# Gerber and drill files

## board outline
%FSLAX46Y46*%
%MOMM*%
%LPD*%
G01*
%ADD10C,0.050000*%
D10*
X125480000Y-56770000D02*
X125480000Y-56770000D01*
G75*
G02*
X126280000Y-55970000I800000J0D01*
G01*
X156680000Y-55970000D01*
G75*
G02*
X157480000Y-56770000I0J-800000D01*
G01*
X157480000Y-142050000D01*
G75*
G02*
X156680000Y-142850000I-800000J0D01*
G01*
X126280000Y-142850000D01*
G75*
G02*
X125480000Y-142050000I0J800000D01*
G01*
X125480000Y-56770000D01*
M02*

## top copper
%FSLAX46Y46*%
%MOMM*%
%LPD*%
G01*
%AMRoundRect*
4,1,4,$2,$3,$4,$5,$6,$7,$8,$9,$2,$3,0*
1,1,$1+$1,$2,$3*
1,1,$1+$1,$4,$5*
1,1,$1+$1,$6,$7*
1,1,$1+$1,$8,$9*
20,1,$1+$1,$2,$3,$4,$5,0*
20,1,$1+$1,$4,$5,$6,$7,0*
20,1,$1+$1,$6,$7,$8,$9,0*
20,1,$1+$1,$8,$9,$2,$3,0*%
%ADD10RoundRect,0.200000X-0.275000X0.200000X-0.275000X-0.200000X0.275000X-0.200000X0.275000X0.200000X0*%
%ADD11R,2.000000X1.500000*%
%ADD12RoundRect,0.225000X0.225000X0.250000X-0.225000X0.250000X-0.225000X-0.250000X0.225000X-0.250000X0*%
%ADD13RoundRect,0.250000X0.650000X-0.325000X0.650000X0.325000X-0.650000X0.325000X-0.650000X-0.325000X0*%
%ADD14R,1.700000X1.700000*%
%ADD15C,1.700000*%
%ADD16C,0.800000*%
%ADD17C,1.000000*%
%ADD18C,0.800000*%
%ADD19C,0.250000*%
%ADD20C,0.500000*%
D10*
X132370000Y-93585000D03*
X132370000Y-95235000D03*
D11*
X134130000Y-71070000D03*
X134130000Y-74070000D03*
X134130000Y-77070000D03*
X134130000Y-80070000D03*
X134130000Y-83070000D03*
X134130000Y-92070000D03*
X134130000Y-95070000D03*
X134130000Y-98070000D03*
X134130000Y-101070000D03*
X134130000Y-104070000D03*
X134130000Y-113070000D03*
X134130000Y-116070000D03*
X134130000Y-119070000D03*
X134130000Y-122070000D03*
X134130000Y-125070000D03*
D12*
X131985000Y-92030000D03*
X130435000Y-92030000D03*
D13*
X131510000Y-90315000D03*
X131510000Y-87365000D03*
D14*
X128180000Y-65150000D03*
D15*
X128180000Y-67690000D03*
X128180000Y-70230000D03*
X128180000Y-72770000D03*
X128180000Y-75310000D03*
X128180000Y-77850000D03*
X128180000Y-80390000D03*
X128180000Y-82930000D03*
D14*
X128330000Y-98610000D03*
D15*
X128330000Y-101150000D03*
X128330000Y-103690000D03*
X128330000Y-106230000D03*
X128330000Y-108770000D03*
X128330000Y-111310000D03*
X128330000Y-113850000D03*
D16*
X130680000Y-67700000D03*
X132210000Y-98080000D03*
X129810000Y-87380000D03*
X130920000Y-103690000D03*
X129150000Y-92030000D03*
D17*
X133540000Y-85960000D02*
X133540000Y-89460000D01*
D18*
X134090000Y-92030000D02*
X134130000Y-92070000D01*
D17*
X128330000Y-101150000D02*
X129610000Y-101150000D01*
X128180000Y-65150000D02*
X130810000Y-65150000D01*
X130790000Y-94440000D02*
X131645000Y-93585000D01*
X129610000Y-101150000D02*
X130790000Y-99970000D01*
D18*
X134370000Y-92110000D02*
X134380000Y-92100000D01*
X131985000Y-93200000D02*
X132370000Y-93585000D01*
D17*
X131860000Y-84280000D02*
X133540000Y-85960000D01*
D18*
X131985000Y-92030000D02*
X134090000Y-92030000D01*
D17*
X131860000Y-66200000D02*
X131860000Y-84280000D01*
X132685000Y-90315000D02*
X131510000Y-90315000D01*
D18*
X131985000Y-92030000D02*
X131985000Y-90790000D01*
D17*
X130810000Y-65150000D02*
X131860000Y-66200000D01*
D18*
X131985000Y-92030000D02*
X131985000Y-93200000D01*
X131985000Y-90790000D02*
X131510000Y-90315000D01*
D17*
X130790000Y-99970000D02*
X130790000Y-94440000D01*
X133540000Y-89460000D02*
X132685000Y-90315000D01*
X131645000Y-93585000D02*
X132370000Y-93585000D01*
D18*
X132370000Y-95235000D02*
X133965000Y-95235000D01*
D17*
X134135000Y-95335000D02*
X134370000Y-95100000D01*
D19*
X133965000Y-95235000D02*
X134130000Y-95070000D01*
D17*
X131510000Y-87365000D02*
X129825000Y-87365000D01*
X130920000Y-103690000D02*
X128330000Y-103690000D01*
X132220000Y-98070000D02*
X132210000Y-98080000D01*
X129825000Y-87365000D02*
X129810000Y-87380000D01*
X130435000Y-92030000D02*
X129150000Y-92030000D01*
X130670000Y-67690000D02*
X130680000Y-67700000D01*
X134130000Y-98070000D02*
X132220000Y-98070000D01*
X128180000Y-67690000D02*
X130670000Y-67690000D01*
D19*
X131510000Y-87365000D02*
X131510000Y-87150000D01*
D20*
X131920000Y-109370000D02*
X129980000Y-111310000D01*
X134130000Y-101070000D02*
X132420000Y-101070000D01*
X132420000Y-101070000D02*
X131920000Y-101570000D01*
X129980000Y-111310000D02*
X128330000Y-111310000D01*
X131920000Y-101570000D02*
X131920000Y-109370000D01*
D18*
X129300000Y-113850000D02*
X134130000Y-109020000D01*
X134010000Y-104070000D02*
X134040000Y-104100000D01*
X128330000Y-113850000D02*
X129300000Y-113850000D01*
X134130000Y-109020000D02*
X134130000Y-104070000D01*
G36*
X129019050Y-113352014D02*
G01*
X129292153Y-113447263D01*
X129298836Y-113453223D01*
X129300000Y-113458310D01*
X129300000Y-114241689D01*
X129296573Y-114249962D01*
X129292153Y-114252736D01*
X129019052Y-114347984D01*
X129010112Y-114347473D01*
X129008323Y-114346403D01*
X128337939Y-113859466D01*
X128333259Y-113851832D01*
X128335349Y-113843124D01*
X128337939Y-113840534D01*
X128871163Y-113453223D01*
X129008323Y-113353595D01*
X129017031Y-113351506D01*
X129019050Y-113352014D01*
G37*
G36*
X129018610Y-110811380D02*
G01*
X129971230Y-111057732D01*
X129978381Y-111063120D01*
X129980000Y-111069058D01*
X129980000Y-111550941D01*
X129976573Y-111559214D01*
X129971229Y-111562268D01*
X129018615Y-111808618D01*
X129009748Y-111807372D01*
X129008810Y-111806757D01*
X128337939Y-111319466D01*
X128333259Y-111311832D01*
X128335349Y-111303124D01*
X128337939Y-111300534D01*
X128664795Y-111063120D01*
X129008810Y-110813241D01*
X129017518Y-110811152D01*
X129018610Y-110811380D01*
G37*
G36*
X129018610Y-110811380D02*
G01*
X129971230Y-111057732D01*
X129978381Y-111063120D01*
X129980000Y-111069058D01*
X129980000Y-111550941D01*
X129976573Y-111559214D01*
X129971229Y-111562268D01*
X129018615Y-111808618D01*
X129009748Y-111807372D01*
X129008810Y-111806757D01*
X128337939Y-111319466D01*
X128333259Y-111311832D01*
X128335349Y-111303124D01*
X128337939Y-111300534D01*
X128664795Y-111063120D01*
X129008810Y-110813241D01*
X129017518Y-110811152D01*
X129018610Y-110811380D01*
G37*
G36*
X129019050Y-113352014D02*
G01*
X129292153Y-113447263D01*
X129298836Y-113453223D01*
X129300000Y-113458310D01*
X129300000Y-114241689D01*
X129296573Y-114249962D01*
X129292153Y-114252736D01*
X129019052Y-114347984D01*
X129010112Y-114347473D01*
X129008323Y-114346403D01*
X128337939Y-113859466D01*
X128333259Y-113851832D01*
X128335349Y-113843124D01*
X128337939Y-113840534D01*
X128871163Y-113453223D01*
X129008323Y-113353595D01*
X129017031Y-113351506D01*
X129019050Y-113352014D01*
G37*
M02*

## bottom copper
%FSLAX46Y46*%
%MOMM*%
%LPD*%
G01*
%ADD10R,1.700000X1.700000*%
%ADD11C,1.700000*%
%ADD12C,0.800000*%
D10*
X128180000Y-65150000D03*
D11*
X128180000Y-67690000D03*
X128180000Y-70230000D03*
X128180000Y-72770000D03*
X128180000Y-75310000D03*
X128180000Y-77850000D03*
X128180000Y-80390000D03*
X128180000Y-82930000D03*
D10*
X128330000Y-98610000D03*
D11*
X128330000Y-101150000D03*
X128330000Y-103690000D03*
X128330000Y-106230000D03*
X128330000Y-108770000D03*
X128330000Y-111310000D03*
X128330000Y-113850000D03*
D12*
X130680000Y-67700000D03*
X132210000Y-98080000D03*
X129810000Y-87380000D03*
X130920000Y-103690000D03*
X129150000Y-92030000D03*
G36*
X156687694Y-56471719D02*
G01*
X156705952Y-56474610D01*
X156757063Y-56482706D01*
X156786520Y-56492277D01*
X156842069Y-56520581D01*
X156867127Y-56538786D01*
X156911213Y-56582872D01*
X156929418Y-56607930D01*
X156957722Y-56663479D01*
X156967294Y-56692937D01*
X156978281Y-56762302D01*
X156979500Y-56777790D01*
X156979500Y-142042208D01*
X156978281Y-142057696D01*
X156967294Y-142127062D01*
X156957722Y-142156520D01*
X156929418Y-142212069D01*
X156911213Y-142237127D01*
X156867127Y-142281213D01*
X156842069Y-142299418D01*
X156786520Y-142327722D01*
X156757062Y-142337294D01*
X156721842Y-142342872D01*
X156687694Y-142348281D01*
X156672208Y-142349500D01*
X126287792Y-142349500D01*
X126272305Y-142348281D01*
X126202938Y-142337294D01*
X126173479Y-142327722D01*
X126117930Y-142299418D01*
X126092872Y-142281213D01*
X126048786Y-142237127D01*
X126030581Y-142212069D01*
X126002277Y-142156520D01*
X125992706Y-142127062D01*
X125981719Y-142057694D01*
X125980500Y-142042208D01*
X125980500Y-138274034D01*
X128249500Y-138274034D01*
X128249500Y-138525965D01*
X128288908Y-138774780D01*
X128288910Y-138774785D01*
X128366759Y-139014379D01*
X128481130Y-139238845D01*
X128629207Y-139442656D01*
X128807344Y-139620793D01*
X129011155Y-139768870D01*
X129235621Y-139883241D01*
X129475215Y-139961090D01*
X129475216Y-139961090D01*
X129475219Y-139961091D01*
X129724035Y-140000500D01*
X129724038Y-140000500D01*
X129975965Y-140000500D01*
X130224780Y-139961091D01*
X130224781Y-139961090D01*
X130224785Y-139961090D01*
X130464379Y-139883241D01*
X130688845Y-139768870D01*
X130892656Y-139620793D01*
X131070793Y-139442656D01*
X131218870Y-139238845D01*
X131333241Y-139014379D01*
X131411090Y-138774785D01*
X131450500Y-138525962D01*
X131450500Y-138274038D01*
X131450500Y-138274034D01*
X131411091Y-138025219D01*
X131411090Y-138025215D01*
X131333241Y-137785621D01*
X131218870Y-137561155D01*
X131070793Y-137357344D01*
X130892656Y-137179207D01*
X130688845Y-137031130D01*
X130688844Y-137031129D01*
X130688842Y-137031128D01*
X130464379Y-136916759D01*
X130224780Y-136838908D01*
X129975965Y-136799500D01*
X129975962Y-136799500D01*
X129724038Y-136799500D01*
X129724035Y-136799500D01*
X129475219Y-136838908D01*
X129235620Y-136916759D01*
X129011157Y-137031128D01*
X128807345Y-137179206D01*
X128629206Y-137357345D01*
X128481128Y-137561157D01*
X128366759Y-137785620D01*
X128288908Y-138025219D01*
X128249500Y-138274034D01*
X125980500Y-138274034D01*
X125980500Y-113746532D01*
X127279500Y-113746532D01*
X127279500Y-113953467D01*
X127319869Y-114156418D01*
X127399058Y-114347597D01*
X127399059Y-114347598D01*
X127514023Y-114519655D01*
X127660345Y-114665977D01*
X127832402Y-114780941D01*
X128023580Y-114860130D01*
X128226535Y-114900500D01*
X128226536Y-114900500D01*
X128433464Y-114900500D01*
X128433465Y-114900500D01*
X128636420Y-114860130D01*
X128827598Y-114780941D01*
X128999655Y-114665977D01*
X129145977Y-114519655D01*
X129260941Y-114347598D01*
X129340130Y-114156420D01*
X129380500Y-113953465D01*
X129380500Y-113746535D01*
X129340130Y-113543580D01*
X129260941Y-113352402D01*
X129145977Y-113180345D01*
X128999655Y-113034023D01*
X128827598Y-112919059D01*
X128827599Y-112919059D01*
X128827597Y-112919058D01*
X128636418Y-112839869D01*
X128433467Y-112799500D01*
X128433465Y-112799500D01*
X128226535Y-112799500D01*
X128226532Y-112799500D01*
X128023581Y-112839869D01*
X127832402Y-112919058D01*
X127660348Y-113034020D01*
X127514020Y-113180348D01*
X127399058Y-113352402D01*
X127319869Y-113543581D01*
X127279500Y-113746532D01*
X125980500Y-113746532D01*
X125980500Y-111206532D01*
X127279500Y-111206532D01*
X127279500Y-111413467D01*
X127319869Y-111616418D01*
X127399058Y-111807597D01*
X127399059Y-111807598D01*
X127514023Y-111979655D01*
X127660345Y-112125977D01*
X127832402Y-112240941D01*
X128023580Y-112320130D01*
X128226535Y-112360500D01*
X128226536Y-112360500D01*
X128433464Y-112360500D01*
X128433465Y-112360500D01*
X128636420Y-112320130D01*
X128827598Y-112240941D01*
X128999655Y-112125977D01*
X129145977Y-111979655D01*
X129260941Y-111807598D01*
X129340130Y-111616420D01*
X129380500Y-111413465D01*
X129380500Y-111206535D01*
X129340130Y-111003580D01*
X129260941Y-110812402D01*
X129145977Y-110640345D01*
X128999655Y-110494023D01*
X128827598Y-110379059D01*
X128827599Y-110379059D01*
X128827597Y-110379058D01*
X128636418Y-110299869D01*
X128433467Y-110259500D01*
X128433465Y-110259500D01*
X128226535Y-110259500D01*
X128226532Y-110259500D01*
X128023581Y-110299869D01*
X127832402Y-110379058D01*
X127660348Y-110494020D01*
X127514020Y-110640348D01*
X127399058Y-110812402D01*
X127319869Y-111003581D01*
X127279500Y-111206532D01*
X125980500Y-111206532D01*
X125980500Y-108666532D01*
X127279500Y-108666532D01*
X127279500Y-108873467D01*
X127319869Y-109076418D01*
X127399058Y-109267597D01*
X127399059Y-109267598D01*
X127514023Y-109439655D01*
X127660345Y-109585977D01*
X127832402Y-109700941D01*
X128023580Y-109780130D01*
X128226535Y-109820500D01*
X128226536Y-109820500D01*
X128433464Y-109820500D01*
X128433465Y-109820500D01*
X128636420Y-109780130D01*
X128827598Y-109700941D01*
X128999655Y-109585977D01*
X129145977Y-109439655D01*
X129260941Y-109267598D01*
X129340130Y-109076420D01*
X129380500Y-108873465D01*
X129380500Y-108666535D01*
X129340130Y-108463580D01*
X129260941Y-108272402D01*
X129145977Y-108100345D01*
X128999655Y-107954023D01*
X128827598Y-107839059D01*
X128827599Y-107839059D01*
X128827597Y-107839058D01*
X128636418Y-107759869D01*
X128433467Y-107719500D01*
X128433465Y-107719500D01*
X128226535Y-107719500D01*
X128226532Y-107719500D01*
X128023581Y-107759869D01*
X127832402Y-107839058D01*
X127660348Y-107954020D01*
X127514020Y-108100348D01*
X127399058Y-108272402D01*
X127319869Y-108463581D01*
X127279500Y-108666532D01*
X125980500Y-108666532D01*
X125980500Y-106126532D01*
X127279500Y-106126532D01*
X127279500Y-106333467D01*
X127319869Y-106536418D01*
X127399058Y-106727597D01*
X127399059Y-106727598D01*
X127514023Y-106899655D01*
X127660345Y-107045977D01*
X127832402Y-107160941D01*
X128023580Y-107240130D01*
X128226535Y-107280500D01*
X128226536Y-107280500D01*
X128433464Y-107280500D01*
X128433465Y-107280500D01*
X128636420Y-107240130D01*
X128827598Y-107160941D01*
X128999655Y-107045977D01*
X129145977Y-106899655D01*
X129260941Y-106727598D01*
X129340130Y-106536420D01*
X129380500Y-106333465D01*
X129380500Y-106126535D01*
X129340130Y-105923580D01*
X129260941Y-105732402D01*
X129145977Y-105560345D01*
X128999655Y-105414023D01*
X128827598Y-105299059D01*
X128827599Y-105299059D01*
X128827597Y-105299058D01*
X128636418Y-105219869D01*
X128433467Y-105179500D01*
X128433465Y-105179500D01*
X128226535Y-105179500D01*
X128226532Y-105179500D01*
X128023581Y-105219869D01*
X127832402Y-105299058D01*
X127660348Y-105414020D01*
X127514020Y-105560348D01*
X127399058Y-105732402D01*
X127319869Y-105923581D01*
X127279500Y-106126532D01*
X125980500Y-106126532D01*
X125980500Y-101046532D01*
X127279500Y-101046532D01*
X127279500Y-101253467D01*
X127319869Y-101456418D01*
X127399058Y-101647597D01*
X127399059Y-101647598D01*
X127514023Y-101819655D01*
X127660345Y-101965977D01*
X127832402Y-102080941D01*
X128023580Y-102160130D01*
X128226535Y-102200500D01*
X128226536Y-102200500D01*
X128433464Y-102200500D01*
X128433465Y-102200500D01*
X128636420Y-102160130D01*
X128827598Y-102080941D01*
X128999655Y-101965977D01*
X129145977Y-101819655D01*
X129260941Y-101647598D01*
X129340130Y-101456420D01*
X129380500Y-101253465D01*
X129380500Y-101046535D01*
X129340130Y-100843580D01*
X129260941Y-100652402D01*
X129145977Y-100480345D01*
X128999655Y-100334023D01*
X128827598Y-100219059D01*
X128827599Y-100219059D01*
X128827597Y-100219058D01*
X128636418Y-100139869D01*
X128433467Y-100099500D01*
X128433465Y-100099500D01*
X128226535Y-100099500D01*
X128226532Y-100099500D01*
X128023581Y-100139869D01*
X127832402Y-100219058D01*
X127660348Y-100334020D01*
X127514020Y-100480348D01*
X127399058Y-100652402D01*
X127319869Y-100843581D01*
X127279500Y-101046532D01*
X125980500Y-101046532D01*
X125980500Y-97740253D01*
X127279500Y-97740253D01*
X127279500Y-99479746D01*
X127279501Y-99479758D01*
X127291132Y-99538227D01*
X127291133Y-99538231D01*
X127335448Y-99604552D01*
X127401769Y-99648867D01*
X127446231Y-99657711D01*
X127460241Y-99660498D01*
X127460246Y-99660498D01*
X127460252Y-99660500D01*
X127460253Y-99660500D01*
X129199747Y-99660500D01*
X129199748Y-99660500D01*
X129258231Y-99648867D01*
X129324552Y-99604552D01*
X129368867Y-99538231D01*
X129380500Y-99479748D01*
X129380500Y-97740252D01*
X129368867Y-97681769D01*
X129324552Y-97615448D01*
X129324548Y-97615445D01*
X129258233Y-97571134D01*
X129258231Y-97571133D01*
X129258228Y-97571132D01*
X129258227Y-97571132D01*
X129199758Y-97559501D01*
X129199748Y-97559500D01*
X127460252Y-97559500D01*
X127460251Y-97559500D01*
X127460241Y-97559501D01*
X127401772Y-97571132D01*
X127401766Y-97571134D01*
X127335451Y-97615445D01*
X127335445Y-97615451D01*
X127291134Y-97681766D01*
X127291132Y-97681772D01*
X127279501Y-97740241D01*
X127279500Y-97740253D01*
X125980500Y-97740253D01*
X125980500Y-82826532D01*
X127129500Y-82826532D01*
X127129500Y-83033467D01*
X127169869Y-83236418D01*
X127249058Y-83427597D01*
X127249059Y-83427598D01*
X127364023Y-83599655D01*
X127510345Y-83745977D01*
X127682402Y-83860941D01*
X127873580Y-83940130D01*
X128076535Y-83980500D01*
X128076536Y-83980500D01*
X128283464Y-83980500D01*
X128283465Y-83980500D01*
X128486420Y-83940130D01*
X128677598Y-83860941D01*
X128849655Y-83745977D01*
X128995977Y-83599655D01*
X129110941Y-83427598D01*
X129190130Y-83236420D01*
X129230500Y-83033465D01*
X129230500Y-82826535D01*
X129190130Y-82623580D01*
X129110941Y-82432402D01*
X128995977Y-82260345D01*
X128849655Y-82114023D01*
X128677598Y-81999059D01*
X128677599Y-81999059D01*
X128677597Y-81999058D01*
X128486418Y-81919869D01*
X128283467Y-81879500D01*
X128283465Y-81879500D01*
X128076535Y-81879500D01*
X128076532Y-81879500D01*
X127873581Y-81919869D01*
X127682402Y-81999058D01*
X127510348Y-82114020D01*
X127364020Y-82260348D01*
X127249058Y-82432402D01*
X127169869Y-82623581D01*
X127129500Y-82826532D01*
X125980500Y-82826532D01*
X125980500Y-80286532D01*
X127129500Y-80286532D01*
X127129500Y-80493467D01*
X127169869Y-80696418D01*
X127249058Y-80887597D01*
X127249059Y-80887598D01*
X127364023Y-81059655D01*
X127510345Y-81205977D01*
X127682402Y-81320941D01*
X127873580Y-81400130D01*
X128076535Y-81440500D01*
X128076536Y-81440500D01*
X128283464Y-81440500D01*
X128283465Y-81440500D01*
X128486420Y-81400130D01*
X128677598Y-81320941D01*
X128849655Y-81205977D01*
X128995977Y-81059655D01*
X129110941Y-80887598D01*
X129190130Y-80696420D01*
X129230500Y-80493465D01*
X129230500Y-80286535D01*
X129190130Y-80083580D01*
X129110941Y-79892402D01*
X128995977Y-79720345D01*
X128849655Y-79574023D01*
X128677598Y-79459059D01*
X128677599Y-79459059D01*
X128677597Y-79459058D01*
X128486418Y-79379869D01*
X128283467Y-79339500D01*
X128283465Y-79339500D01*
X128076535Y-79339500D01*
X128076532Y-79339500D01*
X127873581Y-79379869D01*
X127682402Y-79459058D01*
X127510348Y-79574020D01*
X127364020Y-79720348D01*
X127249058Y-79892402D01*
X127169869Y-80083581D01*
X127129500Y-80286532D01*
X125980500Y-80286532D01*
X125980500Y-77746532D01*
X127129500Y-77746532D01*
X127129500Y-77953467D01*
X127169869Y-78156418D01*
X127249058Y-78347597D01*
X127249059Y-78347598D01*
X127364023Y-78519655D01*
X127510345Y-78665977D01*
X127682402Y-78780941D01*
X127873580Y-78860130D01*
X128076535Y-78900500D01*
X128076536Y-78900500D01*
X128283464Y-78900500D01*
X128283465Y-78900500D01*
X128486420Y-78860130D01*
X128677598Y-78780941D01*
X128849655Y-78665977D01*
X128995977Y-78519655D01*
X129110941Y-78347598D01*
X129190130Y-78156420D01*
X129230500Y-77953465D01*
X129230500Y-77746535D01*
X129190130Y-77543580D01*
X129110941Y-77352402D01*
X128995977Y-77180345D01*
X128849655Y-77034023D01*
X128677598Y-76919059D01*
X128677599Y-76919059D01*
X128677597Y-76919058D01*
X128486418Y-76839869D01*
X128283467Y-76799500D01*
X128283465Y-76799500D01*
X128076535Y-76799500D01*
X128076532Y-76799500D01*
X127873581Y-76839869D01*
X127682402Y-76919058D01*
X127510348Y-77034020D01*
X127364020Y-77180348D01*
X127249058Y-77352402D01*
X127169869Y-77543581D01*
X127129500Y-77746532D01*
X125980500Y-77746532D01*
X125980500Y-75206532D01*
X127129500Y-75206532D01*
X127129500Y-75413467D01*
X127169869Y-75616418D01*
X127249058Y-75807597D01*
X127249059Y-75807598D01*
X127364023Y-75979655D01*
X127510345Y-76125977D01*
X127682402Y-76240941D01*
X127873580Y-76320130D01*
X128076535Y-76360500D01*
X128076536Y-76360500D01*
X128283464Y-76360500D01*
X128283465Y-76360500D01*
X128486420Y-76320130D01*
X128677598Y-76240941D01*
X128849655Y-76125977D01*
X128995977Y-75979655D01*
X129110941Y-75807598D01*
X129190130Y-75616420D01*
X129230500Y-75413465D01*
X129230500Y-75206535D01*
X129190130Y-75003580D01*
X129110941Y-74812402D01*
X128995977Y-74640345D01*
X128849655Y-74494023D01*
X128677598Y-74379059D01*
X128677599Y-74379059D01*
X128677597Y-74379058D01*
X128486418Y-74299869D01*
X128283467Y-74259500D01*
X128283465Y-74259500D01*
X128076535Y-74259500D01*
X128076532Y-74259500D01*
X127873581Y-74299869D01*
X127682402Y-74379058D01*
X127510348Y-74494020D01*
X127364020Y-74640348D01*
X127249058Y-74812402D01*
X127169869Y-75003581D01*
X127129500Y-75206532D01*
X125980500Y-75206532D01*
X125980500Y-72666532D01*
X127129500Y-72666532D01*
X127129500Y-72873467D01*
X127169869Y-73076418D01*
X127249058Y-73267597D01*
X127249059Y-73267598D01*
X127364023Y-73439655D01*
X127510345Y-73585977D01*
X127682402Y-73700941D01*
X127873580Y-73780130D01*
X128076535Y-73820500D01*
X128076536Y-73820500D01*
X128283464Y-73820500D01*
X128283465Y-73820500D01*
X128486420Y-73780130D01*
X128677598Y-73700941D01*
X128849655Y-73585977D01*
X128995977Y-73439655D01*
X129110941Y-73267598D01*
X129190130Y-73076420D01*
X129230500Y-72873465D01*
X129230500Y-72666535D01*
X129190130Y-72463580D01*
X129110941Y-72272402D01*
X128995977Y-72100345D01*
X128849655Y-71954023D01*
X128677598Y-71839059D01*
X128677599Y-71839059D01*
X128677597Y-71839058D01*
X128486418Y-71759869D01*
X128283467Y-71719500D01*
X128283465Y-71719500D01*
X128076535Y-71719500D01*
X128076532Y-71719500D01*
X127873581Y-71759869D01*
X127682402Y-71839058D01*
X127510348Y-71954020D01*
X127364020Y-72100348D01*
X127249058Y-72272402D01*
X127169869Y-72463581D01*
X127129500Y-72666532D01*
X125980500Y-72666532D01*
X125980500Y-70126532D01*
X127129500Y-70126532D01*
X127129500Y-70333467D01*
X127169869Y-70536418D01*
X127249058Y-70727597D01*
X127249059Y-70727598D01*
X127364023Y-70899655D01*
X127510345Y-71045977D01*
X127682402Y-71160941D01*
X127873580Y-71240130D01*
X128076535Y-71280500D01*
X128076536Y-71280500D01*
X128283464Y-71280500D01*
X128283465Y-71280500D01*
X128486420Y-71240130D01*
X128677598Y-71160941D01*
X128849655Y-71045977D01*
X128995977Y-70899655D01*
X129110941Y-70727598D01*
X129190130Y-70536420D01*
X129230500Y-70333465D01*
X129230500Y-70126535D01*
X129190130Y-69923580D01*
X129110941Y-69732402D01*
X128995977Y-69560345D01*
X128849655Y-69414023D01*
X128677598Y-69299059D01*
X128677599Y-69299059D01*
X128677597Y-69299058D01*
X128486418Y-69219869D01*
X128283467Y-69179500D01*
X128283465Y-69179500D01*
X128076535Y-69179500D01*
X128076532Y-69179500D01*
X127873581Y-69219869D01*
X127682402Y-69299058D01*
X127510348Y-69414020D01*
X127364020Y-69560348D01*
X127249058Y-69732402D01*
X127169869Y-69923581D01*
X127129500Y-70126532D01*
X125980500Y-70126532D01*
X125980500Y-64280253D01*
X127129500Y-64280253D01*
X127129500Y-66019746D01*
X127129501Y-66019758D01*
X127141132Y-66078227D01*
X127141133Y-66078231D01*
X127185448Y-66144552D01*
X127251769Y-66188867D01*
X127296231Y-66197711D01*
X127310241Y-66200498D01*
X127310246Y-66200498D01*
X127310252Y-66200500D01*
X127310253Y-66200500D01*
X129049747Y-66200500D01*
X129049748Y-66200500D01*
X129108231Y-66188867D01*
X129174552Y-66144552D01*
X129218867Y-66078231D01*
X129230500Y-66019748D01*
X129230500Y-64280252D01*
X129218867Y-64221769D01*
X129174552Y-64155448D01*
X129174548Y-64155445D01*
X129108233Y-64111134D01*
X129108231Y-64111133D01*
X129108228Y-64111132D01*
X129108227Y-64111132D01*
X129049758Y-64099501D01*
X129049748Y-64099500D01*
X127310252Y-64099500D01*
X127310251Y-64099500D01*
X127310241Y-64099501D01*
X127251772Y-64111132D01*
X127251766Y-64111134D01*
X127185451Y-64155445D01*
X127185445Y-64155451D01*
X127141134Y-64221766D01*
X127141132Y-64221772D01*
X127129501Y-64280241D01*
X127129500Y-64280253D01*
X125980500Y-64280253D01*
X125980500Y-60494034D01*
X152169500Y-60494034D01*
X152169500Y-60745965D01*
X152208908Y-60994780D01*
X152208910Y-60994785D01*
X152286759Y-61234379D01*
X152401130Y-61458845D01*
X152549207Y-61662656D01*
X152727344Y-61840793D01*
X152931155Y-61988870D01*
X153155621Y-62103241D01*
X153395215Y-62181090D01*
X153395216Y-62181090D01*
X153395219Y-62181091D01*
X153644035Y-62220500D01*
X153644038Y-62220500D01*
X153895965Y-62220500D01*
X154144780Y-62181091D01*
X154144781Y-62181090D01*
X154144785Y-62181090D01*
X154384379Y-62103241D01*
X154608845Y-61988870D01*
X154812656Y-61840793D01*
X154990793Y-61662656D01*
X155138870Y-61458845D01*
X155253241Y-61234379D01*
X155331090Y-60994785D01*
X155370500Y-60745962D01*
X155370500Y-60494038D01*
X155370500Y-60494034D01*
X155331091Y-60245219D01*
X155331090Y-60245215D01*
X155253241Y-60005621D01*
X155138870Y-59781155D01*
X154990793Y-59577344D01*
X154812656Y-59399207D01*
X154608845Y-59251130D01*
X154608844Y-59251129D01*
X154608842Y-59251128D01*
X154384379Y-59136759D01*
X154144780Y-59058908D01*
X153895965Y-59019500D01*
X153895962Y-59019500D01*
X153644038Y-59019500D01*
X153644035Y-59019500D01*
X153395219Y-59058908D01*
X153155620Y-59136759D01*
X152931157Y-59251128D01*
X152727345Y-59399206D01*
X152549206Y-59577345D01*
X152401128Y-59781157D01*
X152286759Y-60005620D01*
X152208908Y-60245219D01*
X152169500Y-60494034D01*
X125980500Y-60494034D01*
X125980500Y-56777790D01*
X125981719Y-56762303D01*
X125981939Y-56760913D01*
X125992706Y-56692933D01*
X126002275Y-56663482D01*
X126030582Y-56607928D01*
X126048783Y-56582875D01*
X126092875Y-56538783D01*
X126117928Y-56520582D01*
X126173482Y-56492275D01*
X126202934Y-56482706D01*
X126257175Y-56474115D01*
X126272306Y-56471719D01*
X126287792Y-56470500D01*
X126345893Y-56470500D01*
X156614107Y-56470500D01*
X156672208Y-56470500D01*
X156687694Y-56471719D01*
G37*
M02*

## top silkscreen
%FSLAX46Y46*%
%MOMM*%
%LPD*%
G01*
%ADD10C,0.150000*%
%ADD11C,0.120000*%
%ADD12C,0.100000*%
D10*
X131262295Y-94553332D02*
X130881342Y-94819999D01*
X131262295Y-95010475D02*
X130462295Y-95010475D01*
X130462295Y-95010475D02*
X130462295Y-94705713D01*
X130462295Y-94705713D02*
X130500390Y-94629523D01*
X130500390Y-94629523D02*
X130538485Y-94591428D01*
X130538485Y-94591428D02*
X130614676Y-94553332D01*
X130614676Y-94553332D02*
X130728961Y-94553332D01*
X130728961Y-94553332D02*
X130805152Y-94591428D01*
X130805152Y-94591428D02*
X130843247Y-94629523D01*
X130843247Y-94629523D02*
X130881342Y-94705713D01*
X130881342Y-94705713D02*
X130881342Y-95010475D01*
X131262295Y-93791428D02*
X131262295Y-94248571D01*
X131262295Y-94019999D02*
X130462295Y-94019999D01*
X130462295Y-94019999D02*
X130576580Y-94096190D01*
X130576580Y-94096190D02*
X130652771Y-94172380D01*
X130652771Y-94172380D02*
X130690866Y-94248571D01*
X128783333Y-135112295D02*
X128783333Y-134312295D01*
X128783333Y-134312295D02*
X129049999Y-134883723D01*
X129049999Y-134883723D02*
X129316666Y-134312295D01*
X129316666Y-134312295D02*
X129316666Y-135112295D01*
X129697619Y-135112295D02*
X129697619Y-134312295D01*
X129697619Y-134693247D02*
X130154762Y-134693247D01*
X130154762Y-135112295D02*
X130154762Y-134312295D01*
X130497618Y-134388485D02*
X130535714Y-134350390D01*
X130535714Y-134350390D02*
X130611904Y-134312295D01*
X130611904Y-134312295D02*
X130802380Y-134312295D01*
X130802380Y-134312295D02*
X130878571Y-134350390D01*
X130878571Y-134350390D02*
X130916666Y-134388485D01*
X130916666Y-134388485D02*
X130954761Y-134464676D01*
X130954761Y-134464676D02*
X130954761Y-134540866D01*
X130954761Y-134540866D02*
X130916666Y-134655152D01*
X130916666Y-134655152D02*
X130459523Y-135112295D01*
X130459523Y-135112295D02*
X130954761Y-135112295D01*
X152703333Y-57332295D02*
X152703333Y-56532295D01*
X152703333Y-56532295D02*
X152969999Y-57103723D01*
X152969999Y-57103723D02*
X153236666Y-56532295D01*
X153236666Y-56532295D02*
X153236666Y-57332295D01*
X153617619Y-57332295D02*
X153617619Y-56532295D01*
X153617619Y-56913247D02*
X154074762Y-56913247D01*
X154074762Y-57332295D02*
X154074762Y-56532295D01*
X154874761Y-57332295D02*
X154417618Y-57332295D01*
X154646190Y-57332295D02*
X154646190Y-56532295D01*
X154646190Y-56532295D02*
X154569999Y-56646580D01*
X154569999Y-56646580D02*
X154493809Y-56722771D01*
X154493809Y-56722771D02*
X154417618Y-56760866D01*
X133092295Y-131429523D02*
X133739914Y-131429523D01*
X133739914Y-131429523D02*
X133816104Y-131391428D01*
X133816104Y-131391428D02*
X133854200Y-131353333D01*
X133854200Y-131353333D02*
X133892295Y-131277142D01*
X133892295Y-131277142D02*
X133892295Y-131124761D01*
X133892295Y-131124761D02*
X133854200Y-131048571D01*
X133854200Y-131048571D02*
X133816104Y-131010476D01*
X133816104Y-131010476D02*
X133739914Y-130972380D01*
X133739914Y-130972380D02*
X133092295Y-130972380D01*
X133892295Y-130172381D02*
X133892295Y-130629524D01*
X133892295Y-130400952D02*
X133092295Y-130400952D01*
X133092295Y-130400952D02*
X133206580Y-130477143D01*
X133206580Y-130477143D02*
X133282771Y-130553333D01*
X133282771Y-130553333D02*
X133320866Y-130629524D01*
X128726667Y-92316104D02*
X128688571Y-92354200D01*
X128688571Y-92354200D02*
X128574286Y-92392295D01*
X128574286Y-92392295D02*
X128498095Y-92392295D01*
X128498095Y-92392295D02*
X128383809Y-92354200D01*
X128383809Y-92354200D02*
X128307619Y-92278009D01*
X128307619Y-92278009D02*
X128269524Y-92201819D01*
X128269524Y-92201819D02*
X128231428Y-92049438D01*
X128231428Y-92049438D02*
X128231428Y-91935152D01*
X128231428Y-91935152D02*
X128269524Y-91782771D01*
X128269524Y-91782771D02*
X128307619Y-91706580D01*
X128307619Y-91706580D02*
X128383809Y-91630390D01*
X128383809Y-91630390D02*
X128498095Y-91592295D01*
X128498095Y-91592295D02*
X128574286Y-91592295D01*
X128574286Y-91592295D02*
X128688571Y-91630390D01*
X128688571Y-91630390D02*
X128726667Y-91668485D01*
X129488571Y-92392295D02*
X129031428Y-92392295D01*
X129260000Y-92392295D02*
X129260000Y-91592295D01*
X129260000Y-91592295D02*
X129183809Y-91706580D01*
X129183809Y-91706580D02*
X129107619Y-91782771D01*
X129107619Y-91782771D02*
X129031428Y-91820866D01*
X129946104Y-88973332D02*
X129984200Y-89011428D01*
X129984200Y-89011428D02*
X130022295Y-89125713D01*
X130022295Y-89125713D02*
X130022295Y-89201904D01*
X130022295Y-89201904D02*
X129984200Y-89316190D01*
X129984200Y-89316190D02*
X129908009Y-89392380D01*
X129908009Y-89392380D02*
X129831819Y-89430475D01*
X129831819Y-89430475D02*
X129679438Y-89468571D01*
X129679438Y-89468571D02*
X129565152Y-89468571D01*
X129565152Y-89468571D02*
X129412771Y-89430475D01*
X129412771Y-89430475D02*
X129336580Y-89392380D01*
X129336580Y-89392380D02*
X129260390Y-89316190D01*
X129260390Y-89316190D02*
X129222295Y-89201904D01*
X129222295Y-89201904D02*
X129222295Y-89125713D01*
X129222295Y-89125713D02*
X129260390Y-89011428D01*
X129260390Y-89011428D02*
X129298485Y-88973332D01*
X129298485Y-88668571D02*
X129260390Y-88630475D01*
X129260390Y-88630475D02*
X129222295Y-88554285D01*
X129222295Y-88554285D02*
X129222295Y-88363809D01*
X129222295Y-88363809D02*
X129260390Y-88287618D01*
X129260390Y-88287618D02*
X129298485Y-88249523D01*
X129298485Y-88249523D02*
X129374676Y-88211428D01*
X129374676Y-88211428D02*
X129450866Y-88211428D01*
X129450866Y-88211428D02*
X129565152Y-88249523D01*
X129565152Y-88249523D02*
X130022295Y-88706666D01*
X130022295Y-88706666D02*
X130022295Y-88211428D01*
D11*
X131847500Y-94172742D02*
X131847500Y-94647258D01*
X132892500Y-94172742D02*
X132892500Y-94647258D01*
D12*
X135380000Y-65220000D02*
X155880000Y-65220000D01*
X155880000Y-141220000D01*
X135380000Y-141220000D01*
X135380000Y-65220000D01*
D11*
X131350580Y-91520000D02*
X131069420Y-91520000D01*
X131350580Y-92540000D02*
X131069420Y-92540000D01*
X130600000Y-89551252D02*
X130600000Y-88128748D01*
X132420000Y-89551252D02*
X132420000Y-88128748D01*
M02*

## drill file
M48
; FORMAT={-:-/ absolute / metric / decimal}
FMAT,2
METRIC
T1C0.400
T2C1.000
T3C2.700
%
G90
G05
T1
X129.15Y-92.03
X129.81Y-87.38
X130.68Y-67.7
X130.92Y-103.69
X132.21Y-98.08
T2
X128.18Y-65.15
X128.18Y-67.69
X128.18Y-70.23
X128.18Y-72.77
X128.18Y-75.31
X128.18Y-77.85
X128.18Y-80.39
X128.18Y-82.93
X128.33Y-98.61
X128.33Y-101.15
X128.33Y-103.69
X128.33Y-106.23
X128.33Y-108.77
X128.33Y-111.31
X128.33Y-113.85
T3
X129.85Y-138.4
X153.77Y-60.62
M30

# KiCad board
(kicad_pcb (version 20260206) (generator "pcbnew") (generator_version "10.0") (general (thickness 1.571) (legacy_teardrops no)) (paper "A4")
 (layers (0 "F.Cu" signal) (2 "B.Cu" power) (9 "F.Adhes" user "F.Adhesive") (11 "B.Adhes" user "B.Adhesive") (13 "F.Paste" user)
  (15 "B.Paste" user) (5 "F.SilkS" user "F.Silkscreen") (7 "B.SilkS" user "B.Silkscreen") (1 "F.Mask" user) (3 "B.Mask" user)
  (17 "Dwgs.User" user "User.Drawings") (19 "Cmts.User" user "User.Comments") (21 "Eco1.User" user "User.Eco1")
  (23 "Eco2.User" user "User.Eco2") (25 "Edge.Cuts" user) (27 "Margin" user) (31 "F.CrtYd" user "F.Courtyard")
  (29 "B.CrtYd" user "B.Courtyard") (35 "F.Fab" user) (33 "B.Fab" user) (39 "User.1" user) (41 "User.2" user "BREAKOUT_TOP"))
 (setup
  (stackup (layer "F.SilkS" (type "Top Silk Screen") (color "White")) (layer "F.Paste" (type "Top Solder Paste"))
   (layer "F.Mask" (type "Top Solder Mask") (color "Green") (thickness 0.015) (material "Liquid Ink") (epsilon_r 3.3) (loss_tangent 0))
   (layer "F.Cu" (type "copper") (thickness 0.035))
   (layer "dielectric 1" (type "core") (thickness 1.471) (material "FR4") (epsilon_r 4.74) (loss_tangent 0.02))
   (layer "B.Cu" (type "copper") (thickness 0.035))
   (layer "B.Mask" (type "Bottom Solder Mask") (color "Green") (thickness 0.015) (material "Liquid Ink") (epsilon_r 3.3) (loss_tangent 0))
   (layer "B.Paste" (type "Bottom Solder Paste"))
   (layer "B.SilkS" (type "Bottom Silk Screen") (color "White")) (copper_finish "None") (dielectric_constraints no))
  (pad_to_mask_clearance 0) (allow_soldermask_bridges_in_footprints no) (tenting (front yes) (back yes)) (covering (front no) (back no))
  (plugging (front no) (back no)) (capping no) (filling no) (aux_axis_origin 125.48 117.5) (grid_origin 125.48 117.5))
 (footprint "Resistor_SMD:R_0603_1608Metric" (layer "F.Cu") (at 132.37 94.41 -90)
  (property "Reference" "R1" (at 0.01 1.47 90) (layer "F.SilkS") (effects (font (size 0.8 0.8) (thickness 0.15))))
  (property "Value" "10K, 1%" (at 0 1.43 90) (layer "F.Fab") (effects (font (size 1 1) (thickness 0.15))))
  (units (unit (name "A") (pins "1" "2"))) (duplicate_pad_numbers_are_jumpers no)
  (fp_line (start -0.237258 0.5225) (end 0.237258 0.5225) (stroke (width 0.12) (type solid)) (layer "F.SilkS"))
  (fp_line (start -0.237258 -0.5225) (end 0.237258 -0.5225) (stroke (width 0.12) (type solid)) (layer "F.SilkS"))
  (pad "1" smd roundrect (at -0.825 0 270) (size 0.8 0.95) (layers "F.Cu" "F.Mask" "F.Paste") (roundrect_rratio 0.25) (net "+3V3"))
  (pad "2" smd roundrect (at 0.825 0 270) (size 0.8 0.95) (layers "F.Cu" "F.Mask" "F.Paste") (roundrect_rratio 0.25) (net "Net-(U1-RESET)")))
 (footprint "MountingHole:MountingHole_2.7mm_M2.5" (layer "F.Cu") (at 129.85 138.4)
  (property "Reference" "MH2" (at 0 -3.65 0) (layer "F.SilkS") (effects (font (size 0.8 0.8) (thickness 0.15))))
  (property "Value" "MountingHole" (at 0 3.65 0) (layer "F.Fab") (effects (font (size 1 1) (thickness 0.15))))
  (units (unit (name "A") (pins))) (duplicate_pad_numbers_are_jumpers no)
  (pad "" np_thru_hole circle (at 0 0) (size 2.7 2.7) (drill 2.7) (layers "*.Cu" "*.Mask")))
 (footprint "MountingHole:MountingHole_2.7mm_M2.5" (layer "F.Cu") (at 153.77 60.62)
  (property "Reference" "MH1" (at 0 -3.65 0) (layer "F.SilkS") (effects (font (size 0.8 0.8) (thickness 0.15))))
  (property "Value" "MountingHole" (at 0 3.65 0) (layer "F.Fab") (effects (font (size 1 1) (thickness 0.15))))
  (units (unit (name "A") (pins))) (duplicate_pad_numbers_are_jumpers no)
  (pad "" np_thru_hole circle (at 0 0) (size 2.7 2.7) (drill 2.7) (layers "*.Cu" "*.Mask")))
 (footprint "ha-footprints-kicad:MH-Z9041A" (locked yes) (layer "F.Cu") (at 145.63 103.22 -90)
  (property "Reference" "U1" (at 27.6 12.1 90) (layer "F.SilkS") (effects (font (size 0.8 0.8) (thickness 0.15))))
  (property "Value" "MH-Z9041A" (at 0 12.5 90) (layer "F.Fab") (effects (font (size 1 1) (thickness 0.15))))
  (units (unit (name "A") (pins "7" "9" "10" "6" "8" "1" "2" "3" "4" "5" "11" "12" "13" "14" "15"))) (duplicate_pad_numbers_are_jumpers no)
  (fp_rect (start -38 -10.25) (end 38 10.25) (stroke (width 0.1) (type default)) (fill no) (layer "F.SilkS"))
  (pad "1" smd rect (at -32.15 11.5 270) (size 1.5 2) (layers "F.Cu" "F.Mask" "F.Paste") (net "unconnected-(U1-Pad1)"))
  (pad "2" smd rect (at -29.15 11.5 270) (size 1.5 2) (layers "F.Cu" "F.Mask" "F.Paste") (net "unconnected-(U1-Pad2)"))
  (pad "3" smd rect (at -26.15 11.5 270) (size 1.5 2) (layers "F.Cu" "F.Mask" "F.Paste") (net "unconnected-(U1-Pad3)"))
  (pad "4" smd rect (at -23.15 11.5 270) (size 1.5 2) (layers "F.Cu" "F.Mask" "F.Paste") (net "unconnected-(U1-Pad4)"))
  (pad "5" smd rect (at -20.15 11.5 270) (size 1.5 2) (layers "F.Cu" "F.Mask" "F.Paste") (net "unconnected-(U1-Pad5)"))
  (pad "6" smd rect (at -11.15 11.5 270) (size 1.5 2) (layers "F.Cu" "F.Mask" "F.Paste") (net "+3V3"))
  (pad "7" smd rect (at -8.15 11.5 270) (size 1.5 2) (layers "F.Cu" "F.Mask" "F.Paste") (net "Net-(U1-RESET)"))
  (pad "8" smd rect (at -5.15 11.5 270) (size 1.5 2) (layers "F.Cu" "F.Mask" "F.Paste") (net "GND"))
  (pad "9" smd rect (at -2.15 11.5 270) (size 1.5 2) (layers "F.Cu" "F.Mask" "F.Paste") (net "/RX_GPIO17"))
  (pad "10" smd rect (at 0.85 11.5 270) (size 1.5 2) (layers "F.Cu" "F.Mask" "F.Paste") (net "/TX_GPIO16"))
  (pad "11" smd rect (at 9.85 11.5 270) (size 1.5 2) (layers "F.Cu" "F.Mask" "F.Paste") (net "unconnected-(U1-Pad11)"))
  (pad "12" smd rect (at 12.85 11.5 270) (size 1.5 2) (layers "F.Cu" "F.Mask" "F.Paste") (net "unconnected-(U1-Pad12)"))
  (pad "13" smd rect (at 15.85 11.5 270) (size 1.5 2) (layers "F.Cu" "F.Mask" "F.Paste") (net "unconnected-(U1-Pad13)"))
  (pad "14" smd rect (at 18.85 11.5 270) (size 1.5 2) (layers "F.Cu" "F.Mask" "F.Paste") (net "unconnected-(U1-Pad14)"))
  (pad "15" smd rect (at 21.85 11.5 270) (size 1.5 2) (layers "F.Cu" "F.Mask" "F.Paste") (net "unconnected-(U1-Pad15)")))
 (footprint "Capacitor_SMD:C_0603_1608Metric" (layer "F.Cu") (at 131.21 92.03 180)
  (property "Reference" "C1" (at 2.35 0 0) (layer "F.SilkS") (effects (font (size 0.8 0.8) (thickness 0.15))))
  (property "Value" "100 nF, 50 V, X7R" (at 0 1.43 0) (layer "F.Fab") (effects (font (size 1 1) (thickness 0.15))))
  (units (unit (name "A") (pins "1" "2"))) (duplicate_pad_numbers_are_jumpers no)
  (fp_line (start -0.14058 0.51) (end 0.14058 0.51) (stroke (width 0.12) (type solid)) (layer "F.SilkS"))
  (fp_line (start -0.14058 -0.51) (end 0.14058 -0.51) (stroke (width 0.12) (type solid)) (layer "F.SilkS"))
  (pad "1" smd roundrect (at -0.775 0 180) (size 0.9 0.95) (layers "F.Cu" "F.Mask" "F.Paste") (roundrect_rratio 0.25) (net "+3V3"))
  (pad "2" smd roundrect (at 0.775 0 180) (size 0.9 0.95) (layers "F.Cu" "F.Mask" "F.Paste") (roundrect_rratio 0.25) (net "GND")))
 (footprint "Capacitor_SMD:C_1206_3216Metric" (layer "F.Cu") (at 131.51 88.84 90)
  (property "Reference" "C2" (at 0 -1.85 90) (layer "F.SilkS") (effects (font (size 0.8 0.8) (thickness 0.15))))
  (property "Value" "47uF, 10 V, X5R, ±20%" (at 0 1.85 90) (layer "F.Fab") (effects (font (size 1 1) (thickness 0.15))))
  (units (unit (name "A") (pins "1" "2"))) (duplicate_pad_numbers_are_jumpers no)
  (fp_line (start -0.711252 -0.91) (end 0.711252 -0.91) (stroke (width 0.12) (type solid)) (layer "F.SilkS"))
  (fp_line (start -0.711252 0.91) (end 0.711252 0.91) (stroke (width 0.12) (type solid)) (layer "F.SilkS"))
  (pad "1" smd roundrect (at -1.475 0 90) (size 1.15 1.8) (layers "F.Cu" "F.Mask" "F.Paste") (roundrect_rratio 0.217391) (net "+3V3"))
  (pad "2" smd roundrect (at 1.475 0 90) (size 1.15 1.8) (layers "F.Cu" "F.Mask" "F.Paste") (roundrect_rratio 0.217391) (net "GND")))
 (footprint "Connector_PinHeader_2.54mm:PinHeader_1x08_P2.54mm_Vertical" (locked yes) (layer "B.Cu") (at 128.18 65.15 180)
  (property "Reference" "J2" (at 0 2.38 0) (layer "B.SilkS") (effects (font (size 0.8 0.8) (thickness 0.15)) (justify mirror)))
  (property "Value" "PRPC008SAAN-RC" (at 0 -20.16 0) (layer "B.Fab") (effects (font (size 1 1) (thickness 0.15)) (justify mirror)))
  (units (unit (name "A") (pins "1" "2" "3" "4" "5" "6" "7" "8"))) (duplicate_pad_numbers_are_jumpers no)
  (pad "1" thru_hole rect (at 0 0 180) (size 1.7 1.7) (drill 1) (layers "*.Cu" "*.Mask") (remove_unused_layers no) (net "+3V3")
   (teardrops (best_length_ratio 0.5) (max_length 1) (best_width_ratio 1) (max_width 1) (curved_edges no) (filter_ratio 0.9) (enabled yes)
    (allow_two_segments no) (prefer_zone_connections yes)))
  (pad "2" thru_hole circle (at 0 -2.54 180) (size 1.7 1.7) (drill 1) (layers "*.Cu" "*.Mask") (remove_unused_layers no) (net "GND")
   (teardrops (best_length_ratio 0.5) (max_length 1) (best_width_ratio 1) (max_width 1) (curved_edges no) (filter_ratio 0.9) (enabled yes)
    (allow_two_segments no) (prefer_zone_connections yes)))
  (pad "3" thru_hole circle (at 0 -5.08 180) (size 1.7 1.7) (drill 1) (layers "*.Cu" "*.Mask") (remove_unused_layers no)
   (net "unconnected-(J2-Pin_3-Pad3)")
   (teardrops (best_length_ratio 0.5) (max_length 1) (best_width_ratio 1) (max_width 1) (curved_edges no) (filter_ratio 0.9) (enabled yes)
    (allow_two_segments no) (prefer_zone_connections yes)))
  (pad "4" thru_hole circle (at 0 -7.62 180) (size 1.7 1.7) (drill 1) (layers "*.Cu" "*.Mask") (remove_unused_layers no)
   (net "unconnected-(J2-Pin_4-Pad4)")
   (teardrops (best_length_ratio 0.5) (max_length 1) (best_width_ratio 1) (max_width 1) (curved_edges no) (filter_ratio 0.9) (enabled yes)
    (allow_two_segments no) (prefer_zone_connections yes)))
  (pad "5" thru_hole circle (at 0 -10.16 180) (size 1.7 1.7) (drill 1) (layers "*.Cu" "*.Mask") (remove_unused_layers no)
   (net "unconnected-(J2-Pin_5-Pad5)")
   (teardrops (best_length_ratio 0.5) (max_length 1) (best_width_ratio 1) (max_width 1) (curved_edges no) (filter_ratio 0.9) (enabled yes)
    (allow_two_segments no) (prefer_zone_connections yes)))
  (pad "6" thru_hole circle (at 0 -12.7 180) (size 1.7 1.7) (drill 1) (layers "*.Cu" "*.Mask") (remove_unused_layers no)
   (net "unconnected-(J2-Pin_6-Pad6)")
   (teardrops (best_length_ratio 0.5) (max_length 1) (best_width_ratio 1) (max_width 1) (curved_edges no) (filter_ratio 0.9) (enabled yes)
    (allow_two_segments no) (prefer_zone_connections yes)))
  (pad "7" thru_hole circle (at 0 -15.24 180) (size 1.7 1.7) (drill 1) (layers "*.Cu" "*.Mask") (remove_unused_layers no)
   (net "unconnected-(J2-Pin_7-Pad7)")
   (teardrops (best_length_ratio 0.5) (max_length 1) (best_width_ratio 1) (max_width 1) (curved_edges no) (filter_ratio 0.9) (enabled yes)
    (allow_two_segments no) (prefer_zone_connections yes)))
  (pad "8" thru_hole circle (at 0 -17.78 180) (size 1.7 1.7) (drill 1) (layers "*.Cu" "*.Mask") (remove_unused_layers no)
   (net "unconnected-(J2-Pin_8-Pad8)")
   (teardrops (best_length_ratio 0.5) (max_length 1) (best_width_ratio 1) (max_width 1) (curved_edges no) (filter_ratio 0.9) (enabled yes)
    (allow_two_segments no) (prefer_zone_connections yes))))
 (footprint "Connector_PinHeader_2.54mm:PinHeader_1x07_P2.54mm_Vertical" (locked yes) (layer "B.Cu") (at 128.33 98.61 180)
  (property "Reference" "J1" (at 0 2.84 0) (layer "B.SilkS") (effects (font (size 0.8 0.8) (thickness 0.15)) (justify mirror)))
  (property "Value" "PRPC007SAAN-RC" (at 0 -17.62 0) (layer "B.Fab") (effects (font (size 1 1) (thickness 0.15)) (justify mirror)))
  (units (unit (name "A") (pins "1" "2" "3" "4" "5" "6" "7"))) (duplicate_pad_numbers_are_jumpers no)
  (pad "1" thru_hole rect (at 0 0 180) (size 1.7 1.7) (drill 1) (layers "*.Cu" "*.Mask") (remove_unused_layers no)
   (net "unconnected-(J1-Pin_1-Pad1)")
   (teardrops (best_length_ratio 0.5) (max_length 1) (best_width_ratio 1) (max_width 1) (curved_edges no) (filter_ratio 0.9) (enabled yes)
    (allow_two_segments no) (prefer_zone_connections yes)))
  (pad "2" thru_hole circle (at 0 -2.54 180) (size 1.7 1.7) (drill 1) (layers "*.Cu" "*.Mask") (remove_unused_layers no) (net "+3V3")
   (teardrops (best_length_ratio 0.5) (max_length 1) (best_width_ratio 1) (max_width 1) (curved_edges no) (filter_ratio 0.9) (enabled yes)
    (allow_two_segments no) (prefer_zone_connections yes)))
  (pad "3" thru_hole circle (at 0 -5.08 180) (size 1.7 1.7) (drill 1) (layers "*.Cu" "*.Mask") (remove_unused_layers no) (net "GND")
   (teardrops (best_length_ratio 0.5) (max_length 1) (best_width_ratio 1) (max_width 1) (curved_edges no) (filter_ratio 0.9) (enabled yes)
    (allow_two_segments no) (prefer_zone_connections yes)))
  (pad "4" thru_hole circle (at 0 -7.62 180) (size 1.7 1.7) (drill 1) (layers "*.Cu" "*.Mask") (remove_unused_layers no)
   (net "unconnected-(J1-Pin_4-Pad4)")
   (teardrops (best_length_ratio 0.5) (max_length 1) (best_width_ratio 1) (max_width 1) (curved_edges no) (filter_ratio 0.9) (enabled yes)
    (allow_two_segments no) (prefer_zone_connections yes)))
  (pad "5" thru_hole circle (at 0 -10.16 180) (size 1.7 1.7) (drill 1) (layers "*.Cu" "*.Mask") (remove_unused_layers no)
   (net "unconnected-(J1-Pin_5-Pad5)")
   (teardrops (best_length_ratio 0.5) (max_length 1) (best_width_ratio 1) (max_width 1) (curved_edges no) (filter_ratio 0.9) (enabled yes)
    (allow_two_segments no) (prefer_zone_connections yes)))
  (pad "6" thru_hole circle (at 0 -12.7 180) (size 1.7 1.7) (drill 1) (layers "*.Cu" "*.Mask") (remove_unused_layers no) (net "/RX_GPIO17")
   (teardrops (best_length_ratio 0.5) (max_length 1) (best_width_ratio 1) (max_width 1) (curved_edges no) (filter_ratio 0.9) (enabled yes)
    (allow_two_segments no) (prefer_zone_connections yes)))
  (pad "7" thru_hole circle (at 0 -15.24 180) (size 1.7 1.7) (drill 1) (layers "*.Cu" "*.Mask") (remove_unused_layers no) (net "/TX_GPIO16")
   (teardrops (best_length_ratio 0.5) (max_length 1) (best_width_ratio 1) (max_width 1) (curved_edges no) (filter_ratio 0.9) (enabled yes)
    (allow_two_segments no) (prefer_zone_connections yes))))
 (gr_rect (start 125.48 55.97) (end 157.48 142.85) (radius 0.8) (stroke (width 0.05) (type solid)) (fill no) (layer "Edge.Cuts"))
 (segment (start 133.54 85.96) (end 133.54 89.46) (width 1) (layer "F.Cu") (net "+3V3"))
 (segment (start 134.09 92.03) (end 134.13 92.07) (width 0.8) (layer "F.Cu") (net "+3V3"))
 (segment (start 128.33 101.15) (end 129.61 101.15) (width 1) (layer "F.Cu") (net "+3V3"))
 (segment (start 128.18 65.15) (end 130.81 65.15) (width 1) (layer "F.Cu") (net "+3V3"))
 (segment (start 130.79 94.44) (end 131.645 93.585) (width 1) (layer "F.Cu") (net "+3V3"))
 (segment (start 129.61 101.15) (end 130.79 99.97) (width 1) (layer "F.Cu") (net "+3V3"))
 (segment (start 134.37 92.11) (end 134.38 92.1) (width 0.8) (layer "F.Cu") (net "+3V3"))
 (segment (start 131.985 93.2) (end 132.37 93.585) (width 0.8) (layer "F.Cu") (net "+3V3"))
 (segment (start 131.86 84.28) (end 133.54 85.96) (width 1) (layer "F.Cu") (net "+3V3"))
 (segment (start 131.985 92.03) (end 134.09 92.03) (width 0.8) (layer "F.Cu") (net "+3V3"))
 (segment (start 131.86 66.2) (end 131.86 84.28) (width 1) (layer "F.Cu") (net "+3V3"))
 (segment (start 132.685 90.315) (end 131.51 90.315) (width 1) (layer "F.Cu") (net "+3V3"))
 (segment (start 131.985 92.03) (end 131.985 90.79) (width 0.8) (layer "F.Cu") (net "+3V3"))
 (segment (start 130.81 65.15) (end 131.86 66.2) (width 1) (layer "F.Cu") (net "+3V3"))
 (segment (start 131.985 92.03) (end 131.985 93.2) (width 0.8) (layer "F.Cu") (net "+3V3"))
 (segment (start 131.985 90.79) (end 131.51 90.315) (width 0.8) (layer "F.Cu") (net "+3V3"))
 (segment (start 130.79 99.97) (end 130.79 94.44) (width 1) (layer "F.Cu") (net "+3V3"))
 (segment (start 133.54 89.46) (end 132.685 90.315) (width 1) (layer "F.Cu") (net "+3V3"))
 (segment (start 131.645 93.585) (end 132.37 93.585) (width 1) (layer "F.Cu") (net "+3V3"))
 (segment (start 132.37 95.235) (end 133.965 95.235) (width 0.8) (layer "F.Cu") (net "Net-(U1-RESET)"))
 (segment (start 134.135 95.335) (end 134.37 95.1) (width 1) (layer "F.Cu") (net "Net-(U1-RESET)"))
 (segment (start 133.965 95.235) (end 134.13 95.07) (width 0.25) (layer "F.Cu") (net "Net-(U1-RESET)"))
 (segment (start 131.51 87.365) (end 129.825 87.365) (width 1) (layer "F.Cu") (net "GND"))
 (segment (start 130.92 103.69) (end 128.33 103.69) (width 1) (layer "F.Cu") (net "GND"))
 (segment (start 132.22 98.07) (end 132.21 98.08) (width 1) (layer "F.Cu") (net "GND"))
 (segment (start 129.825 87.365) (end 129.81 87.38) (width 1) (layer "F.Cu") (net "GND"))
 (segment (start 130.435 92.03) (end 129.15 92.03) (width 1) (layer "F.Cu") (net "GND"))
 (segment (start 130.67 67.69) (end 130.68 67.7) (width 1) (layer "F.Cu") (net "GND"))
 (segment (start 134.13 98.07) (end 132.22 98.07) (width 1) (layer "F.Cu") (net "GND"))
 (segment (start 128.18 67.69) (end 130.67 67.69) (width 1) (layer "F.Cu") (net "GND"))
 (segment (start 131.51 87.365) (end 131.51 87.15) (width 0.25) (layer "F.Cu") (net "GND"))
 (via (at 130.68 67.7) (size 0.8) (drill 0.4) (layers "F.Cu" "B.Cu") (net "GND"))
 (via (at 132.21 98.08) (size 0.8) (drill 0.4) (layers "F.Cu" "B.Cu") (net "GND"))
 (via (at 129.81 87.38) (size 0.8) (drill 0.4) (layers "F.Cu" "B.Cu") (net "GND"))
 (via (at 130.92 103.69) (size 0.8) (drill 0.4) (layers "F.Cu" "B.Cu") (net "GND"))
 (via (at 129.15 92.03) (size 0.8) (drill 0.4) (layers "F.Cu" "B.Cu") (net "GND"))
 (segment (start 131.92 109.37) (end 129.98 111.31) (width 0.5) (layer "F.Cu") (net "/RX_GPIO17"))
 (segment (start 134.13 101.07) (end 132.42 101.07) (width 0.5) (layer "F.Cu") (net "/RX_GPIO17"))
 (segment (start 132.42 101.07) (end 131.92 101.57) (width 0.5) (layer "F.Cu") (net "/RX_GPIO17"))
 (segment (start 129.98 111.31) (end 128.33 111.31) (width 0.5) (layer "F.Cu") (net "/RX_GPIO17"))
 (segment (start 131.92 101.57) (end 131.92 109.37) (width 0.5) (layer "F.Cu") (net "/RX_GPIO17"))
 (segment (start 129.3 113.85) (end 134.13 109.02) (width 0.8) (layer "F.Cu") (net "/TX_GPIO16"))
 (segment (start 134.01 104.07) (end 134.04 104.1) (width 0.8) (layer "F.Cu") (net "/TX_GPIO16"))
 (segment (start 128.33 113.85) (end 129.3 113.85) (width 0.8) (layer "F.Cu") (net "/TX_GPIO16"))
 (segment (start 134.13 109.02) (end 134.13 104.07) (width 0.8) (layer "F.Cu") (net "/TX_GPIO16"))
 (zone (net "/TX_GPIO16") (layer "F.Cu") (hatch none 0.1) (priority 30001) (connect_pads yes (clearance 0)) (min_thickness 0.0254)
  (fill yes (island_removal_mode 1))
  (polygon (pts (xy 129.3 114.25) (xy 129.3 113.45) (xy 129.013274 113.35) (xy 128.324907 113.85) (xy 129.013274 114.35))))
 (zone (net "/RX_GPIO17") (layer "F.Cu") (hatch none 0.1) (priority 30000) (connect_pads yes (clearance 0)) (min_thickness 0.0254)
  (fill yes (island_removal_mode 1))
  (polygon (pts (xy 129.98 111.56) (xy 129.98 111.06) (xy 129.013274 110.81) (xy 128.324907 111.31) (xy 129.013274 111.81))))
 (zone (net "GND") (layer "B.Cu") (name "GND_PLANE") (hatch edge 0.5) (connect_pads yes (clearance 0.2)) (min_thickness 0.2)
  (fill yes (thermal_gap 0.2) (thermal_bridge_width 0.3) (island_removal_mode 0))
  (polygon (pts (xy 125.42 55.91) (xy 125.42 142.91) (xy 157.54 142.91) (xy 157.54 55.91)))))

